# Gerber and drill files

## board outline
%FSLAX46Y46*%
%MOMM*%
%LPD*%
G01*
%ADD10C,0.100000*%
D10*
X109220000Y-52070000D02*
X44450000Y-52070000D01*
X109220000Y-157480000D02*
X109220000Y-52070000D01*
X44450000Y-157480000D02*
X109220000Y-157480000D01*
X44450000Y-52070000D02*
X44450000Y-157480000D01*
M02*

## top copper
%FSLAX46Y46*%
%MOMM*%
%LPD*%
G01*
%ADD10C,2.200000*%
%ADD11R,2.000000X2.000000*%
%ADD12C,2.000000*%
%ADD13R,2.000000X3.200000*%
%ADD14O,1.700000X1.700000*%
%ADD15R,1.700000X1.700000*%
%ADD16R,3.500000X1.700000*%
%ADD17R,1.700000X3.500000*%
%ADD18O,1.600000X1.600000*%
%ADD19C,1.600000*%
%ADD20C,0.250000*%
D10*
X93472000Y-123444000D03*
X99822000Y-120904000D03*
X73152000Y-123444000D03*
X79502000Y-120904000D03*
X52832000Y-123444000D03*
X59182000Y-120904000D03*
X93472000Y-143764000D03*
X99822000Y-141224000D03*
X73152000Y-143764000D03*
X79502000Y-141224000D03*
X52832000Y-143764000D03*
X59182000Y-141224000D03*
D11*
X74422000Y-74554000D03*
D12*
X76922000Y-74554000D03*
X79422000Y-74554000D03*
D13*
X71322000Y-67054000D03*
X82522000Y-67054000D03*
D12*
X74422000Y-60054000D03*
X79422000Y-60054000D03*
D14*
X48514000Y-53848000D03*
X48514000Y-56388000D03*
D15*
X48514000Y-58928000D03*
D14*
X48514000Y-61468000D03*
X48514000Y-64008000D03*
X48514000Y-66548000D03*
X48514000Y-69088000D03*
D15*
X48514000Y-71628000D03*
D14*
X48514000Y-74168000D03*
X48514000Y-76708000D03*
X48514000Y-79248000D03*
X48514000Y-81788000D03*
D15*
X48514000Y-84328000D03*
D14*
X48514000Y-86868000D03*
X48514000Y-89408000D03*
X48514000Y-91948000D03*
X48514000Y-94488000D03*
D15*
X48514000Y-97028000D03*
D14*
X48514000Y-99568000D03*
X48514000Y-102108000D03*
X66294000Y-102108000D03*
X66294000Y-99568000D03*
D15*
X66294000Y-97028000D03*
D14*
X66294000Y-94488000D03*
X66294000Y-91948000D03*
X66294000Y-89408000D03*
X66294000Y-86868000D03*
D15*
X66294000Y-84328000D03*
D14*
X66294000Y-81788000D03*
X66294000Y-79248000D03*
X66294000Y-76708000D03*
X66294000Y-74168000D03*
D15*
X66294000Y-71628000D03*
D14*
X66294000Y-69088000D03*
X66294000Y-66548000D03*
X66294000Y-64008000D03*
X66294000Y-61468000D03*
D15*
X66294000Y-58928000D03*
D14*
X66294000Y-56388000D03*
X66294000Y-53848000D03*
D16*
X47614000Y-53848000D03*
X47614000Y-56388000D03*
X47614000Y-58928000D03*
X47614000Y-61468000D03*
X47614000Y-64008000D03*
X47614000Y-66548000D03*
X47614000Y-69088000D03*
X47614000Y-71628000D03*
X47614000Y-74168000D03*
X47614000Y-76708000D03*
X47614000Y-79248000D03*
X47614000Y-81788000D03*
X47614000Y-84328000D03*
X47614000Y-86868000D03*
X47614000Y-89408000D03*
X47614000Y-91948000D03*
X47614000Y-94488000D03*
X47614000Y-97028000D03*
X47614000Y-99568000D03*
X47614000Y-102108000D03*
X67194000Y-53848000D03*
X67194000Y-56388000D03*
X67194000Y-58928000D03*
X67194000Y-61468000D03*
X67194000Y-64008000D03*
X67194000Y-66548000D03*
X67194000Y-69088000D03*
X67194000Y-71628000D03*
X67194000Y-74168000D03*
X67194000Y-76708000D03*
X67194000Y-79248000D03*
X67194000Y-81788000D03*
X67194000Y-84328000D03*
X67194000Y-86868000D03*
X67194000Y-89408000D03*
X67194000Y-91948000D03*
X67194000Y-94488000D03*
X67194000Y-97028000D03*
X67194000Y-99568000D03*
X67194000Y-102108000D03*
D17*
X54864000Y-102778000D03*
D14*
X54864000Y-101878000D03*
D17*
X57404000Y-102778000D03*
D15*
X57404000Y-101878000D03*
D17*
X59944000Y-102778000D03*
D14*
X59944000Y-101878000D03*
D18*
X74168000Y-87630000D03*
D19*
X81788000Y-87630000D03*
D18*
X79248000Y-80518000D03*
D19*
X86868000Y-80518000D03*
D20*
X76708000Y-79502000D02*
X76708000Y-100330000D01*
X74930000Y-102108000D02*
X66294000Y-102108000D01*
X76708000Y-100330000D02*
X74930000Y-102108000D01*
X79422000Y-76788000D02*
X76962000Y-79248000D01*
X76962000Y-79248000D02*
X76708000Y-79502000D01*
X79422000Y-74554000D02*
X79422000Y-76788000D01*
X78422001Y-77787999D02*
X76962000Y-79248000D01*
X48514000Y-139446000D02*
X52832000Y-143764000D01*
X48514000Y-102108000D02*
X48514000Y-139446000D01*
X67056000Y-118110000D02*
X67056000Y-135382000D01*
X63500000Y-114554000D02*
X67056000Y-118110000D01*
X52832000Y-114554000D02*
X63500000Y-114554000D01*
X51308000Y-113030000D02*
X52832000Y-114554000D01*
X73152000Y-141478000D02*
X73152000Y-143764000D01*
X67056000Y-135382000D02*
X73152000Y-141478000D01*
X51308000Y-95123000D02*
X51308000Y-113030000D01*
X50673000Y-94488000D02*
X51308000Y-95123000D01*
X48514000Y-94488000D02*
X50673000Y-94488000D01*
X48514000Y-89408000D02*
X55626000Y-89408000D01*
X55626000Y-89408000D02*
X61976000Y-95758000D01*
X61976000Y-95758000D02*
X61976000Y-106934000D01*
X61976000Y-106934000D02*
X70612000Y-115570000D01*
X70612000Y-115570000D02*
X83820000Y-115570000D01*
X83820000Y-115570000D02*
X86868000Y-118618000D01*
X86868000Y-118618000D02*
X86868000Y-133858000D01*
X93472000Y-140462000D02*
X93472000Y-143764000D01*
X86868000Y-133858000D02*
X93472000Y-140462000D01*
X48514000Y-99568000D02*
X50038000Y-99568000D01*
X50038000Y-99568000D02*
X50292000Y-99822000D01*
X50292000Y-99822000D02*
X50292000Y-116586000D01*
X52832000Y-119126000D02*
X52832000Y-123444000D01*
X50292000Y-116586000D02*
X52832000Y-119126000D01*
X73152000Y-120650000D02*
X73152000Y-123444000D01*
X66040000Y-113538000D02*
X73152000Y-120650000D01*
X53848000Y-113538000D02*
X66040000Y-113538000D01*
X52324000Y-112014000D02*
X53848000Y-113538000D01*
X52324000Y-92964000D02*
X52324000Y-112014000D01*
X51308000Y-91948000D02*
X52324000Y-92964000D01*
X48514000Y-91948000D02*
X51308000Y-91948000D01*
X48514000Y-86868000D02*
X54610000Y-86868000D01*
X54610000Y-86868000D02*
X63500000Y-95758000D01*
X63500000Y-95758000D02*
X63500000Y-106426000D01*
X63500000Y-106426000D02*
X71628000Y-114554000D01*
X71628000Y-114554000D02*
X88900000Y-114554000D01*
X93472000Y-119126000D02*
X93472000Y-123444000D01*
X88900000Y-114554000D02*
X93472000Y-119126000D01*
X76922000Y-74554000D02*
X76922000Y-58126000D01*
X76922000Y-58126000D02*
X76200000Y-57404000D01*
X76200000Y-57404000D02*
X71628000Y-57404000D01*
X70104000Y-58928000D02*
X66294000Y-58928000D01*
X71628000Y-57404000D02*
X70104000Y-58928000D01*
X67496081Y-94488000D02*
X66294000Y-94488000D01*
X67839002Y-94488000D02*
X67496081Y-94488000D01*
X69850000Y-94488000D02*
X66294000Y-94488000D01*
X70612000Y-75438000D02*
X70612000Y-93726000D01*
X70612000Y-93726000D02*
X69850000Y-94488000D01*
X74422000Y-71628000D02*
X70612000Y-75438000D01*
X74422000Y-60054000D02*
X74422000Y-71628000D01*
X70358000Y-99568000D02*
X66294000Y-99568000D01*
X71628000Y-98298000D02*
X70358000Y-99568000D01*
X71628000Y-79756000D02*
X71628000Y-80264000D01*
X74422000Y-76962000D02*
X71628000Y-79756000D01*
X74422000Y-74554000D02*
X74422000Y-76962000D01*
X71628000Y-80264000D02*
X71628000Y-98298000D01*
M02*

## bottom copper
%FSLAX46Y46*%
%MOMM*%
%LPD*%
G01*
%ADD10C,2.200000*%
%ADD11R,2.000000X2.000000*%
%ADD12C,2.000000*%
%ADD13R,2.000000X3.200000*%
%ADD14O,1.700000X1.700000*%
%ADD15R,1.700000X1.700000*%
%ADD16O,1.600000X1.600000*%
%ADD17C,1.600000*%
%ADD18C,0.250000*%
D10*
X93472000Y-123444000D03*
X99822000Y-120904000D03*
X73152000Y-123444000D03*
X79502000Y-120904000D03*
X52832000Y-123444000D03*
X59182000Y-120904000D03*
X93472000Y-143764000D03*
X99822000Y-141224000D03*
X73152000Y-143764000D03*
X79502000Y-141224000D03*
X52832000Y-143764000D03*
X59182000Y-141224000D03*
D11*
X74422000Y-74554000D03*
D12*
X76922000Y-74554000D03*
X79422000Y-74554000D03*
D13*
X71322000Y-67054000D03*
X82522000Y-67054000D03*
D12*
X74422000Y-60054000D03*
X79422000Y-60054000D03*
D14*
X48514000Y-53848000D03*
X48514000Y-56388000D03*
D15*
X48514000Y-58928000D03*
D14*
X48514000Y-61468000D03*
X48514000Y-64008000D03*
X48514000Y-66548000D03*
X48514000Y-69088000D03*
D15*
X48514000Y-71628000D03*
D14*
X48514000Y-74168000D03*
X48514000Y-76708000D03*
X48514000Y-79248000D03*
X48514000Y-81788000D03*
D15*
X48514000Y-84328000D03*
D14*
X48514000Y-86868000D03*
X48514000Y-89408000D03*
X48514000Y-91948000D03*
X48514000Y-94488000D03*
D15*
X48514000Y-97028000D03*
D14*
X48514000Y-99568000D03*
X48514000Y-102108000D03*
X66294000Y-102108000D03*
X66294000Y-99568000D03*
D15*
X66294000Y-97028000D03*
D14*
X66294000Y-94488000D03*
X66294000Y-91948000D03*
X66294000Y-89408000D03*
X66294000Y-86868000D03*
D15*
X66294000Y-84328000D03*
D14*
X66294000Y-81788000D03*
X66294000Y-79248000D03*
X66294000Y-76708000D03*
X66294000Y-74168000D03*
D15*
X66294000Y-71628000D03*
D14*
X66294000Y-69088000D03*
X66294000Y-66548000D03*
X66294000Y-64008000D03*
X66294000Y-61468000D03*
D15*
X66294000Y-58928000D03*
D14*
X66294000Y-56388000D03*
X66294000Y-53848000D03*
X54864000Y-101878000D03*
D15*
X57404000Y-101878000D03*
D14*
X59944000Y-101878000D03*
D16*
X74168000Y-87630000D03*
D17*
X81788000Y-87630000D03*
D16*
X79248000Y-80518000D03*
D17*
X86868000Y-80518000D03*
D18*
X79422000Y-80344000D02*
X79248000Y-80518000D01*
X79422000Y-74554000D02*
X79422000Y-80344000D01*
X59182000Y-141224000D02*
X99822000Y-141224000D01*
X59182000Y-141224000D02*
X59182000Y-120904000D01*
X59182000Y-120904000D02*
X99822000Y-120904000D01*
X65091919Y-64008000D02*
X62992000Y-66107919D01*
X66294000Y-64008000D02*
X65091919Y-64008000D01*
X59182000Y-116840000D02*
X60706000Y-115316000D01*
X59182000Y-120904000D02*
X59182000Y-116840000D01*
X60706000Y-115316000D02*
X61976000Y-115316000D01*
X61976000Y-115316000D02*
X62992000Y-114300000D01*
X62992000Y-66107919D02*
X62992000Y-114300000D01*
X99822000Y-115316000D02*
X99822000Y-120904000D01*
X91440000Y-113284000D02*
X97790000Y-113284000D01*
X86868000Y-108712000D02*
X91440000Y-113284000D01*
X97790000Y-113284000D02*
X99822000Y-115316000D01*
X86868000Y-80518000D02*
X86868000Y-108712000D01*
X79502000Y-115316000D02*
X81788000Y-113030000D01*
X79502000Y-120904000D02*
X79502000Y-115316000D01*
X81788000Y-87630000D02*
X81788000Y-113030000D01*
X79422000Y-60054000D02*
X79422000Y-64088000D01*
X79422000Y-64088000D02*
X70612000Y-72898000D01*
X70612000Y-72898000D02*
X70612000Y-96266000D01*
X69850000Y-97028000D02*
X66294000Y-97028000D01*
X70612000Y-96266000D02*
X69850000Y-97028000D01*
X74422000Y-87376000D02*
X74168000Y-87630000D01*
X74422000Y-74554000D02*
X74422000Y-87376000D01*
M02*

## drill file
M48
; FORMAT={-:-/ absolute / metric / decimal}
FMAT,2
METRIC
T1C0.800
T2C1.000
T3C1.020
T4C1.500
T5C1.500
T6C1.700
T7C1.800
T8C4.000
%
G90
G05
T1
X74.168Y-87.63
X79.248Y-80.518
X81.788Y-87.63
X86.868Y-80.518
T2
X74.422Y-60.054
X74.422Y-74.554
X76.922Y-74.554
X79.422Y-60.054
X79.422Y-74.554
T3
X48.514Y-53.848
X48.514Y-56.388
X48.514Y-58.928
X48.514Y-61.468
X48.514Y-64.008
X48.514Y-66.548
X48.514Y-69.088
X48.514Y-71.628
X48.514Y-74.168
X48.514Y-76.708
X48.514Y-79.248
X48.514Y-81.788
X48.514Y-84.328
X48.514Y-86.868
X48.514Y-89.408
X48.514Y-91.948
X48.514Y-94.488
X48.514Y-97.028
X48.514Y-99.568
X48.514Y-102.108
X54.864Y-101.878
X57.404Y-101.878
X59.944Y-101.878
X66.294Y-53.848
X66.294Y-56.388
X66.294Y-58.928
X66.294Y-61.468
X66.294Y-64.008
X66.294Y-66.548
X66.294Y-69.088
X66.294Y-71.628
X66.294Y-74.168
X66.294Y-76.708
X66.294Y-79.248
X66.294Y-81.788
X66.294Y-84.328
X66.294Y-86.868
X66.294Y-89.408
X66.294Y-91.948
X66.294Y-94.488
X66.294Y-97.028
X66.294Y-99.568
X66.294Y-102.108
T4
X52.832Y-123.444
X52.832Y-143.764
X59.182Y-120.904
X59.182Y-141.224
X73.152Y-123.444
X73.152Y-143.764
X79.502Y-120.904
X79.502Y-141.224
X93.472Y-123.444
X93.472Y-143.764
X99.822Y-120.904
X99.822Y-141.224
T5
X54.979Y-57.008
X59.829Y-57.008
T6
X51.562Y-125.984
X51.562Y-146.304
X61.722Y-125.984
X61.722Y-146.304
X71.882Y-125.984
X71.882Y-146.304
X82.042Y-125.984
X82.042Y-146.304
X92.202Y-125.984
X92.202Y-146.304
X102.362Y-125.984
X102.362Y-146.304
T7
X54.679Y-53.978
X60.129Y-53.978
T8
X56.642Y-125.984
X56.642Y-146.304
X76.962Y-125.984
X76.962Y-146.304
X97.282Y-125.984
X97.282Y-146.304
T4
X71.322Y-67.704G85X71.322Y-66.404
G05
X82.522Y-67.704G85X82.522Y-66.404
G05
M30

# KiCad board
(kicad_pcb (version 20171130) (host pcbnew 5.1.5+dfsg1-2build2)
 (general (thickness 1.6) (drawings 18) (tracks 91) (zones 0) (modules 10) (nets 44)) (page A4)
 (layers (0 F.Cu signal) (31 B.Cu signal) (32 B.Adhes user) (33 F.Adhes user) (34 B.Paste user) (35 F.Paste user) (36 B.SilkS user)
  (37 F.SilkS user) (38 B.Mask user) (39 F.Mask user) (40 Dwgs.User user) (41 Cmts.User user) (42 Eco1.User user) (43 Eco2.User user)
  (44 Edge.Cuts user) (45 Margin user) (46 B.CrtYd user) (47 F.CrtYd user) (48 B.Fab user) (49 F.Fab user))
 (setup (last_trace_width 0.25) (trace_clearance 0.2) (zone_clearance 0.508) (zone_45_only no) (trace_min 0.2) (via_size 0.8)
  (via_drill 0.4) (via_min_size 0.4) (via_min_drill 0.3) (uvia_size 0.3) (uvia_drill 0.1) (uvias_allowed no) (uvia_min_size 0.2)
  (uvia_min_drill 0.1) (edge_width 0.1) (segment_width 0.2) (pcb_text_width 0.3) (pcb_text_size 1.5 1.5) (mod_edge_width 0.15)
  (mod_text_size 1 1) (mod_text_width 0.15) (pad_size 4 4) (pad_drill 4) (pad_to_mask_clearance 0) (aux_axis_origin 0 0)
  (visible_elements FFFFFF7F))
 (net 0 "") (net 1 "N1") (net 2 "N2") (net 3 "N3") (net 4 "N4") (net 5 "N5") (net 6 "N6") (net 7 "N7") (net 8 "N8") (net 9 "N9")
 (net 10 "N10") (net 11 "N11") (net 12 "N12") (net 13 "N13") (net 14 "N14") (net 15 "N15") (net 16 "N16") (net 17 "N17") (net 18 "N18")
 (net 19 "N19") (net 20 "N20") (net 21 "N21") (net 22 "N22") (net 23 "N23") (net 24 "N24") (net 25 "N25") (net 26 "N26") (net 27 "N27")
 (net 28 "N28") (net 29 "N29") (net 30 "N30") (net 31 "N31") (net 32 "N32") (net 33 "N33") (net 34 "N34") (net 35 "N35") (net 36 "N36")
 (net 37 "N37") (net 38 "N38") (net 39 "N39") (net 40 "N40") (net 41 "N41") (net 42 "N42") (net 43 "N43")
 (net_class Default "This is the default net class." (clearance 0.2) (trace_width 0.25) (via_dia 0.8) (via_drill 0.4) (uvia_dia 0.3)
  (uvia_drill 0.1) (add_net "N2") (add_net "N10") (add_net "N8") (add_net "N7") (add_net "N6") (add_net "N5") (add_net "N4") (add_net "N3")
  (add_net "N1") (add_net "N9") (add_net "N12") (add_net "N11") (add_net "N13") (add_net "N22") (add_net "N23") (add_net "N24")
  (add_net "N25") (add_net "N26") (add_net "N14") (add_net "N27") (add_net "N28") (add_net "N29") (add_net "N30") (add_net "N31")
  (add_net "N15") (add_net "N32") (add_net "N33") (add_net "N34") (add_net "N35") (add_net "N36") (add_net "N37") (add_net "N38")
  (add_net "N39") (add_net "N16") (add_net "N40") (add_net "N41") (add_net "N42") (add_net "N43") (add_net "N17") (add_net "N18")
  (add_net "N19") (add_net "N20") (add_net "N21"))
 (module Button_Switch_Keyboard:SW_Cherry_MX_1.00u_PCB (layer F.Cu) (at 99.822 120.904)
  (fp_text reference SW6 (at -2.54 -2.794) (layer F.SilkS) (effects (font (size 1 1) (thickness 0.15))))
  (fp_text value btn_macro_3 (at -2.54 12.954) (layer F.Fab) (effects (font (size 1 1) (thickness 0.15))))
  (pad "" np_thru_hole circle (at 2.54 5.08) (size 1.7 1.7) (drill 1.7) (layers *.Cu *.Mask))
  (pad "" np_thru_hole circle (at -7.62 5.08) (size 1.7 1.7) (drill 1.7) (layers *.Cu *.Mask))
  (pad "" np_thru_hole circle (at -2.54 5.08) (size 4 4) (drill 4) (layers *.Cu *.Mask))
  (pad 2 thru_hole circle (at -6.35 2.54) (size 2.2 2.2) (drill 1.5) (layers *.Cu *.Mask) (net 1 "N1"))
  (pad 1 thru_hole circle (at 0 0) (size 2.2 2.2) (drill 1.5) (layers *.Cu *.Mask) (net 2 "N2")))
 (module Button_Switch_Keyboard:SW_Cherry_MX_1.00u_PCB (layer F.Cu) (at 79.502 120.904)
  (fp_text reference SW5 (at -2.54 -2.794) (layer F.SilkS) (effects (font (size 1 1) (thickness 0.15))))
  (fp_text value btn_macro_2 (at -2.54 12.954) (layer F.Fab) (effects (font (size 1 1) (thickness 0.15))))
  (pad "" np_thru_hole circle (at 2.54 5.08) (size 1.7 1.7) (drill 1.7) (layers *.Cu *.Mask))
  (pad "" np_thru_hole circle (at -7.62 5.08) (size 1.7 1.7) (drill 1.7) (layers *.Cu *.Mask))
  (pad "" np_thru_hole circle (at -2.54 5.08) (size 4 4) (drill 4) (layers *.Cu *.Mask))
  (pad 2 thru_hole circle (at -6.35 2.54) (size 2.2 2.2) (drill 1.5) (layers *.Cu *.Mask) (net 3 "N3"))
  (pad 1 thru_hole circle (at 0 0) (size 2.2 2.2) (drill 1.5) (layers *.Cu *.Mask) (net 2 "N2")))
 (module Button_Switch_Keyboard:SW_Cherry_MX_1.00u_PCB (layer F.Cu) (at 59.182 120.904)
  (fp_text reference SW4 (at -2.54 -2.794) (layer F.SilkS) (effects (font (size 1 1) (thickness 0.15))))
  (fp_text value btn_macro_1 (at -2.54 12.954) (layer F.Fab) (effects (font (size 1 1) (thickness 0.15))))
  (pad "" np_thru_hole circle (at 2.54 5.08) (size 1.7 1.7) (drill 1.7) (layers *.Cu *.Mask))
  (pad "" np_thru_hole circle (at -7.62 5.08) (size 1.7 1.7) (drill 1.7) (layers *.Cu *.Mask))
  (pad "" np_thru_hole circle (at -2.54 5.08) (size 4 4) (drill 4) (layers *.Cu *.Mask))
  (pad 2 thru_hole circle (at -6.35 2.54) (size 2.2 2.2) (drill 1.5) (layers *.Cu *.Mask) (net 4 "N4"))
  (pad 1 thru_hole circle (at 0 0) (size 2.2 2.2) (drill 1.5) (layers *.Cu *.Mask) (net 2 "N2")))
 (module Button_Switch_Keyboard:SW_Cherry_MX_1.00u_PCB (layer F.Cu) (at 99.822 141.224)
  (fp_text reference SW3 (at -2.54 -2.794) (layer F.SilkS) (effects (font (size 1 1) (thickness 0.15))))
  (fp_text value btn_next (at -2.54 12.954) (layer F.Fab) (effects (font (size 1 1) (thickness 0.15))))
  (pad "" np_thru_hole circle (at 2.54 5.08) (size 1.7 1.7) (drill 1.7) (layers *.Cu *.Mask))
  (pad "" np_thru_hole circle (at -7.62 5.08) (size 1.7 1.7) (drill 1.7) (layers *.Cu *.Mask))
  (pad "" np_thru_hole circle (at -2.54 5.08) (size 4 4) (drill 4) (layers *.Cu *.Mask))
  (pad 2 thru_hole circle (at -6.35 2.54) (size 2.2 2.2) (drill 1.5) (layers *.Cu *.Mask) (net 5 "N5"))
  (pad 1 thru_hole circle (at 0 0) (size 2.2 2.2) (drill 1.5) (layers *.Cu *.Mask) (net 2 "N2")))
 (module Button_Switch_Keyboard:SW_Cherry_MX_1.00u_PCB (layer F.Cu) (at 79.502 141.224)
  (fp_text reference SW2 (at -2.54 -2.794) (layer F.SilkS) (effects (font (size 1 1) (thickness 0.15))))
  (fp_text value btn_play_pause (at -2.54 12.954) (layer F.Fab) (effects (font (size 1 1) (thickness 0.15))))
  (pad "" np_thru_hole circle (at 2.54 5.08) (size 1.7 1.7) (drill 1.7) (layers *.Cu *.Mask))
  (pad "" np_thru_hole circle (at -7.62 5.08) (size 1.7 1.7) (drill 1.7) (layers *.Cu *.Mask))
  (pad "" np_thru_hole circle (at -2.54 5.08) (size 4 4) (drill 4) (layers *.Cu *.Mask))
  (pad 2 thru_hole circle (at -6.35 2.54) (size 2.2 2.2) (drill 1.5) (layers *.Cu *.Mask) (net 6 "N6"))
  (pad 1 thru_hole circle (at 0 0) (size 2.2 2.2) (drill 1.5) (layers *.Cu *.Mask) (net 2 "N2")))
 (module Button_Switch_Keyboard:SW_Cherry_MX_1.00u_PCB (layer F.Cu) (at 59.182 141.224)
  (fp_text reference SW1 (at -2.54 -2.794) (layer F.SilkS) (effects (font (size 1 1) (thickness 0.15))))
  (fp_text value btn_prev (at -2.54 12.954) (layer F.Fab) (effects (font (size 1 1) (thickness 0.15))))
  (pad "" np_thru_hole circle (at 2.54 5.08) (size 1.7 1.7) (drill 1.7) (layers *.Cu *.Mask))
  (pad "" np_thru_hole circle (at -7.62 5.08) (size 1.7 1.7) (drill 1.7) (layers *.Cu *.Mask))
  (pad "" np_thru_hole circle (at -2.54 5.08) (size 4 4) (drill 4) (layers *.Cu *.Mask))
  (pad 2 thru_hole circle (at -6.35 2.54) (size 2.2 2.2) (drill 1.5) (layers *.Cu *.Mask) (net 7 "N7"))
  (pad 1 thru_hole circle (at 0 0) (size 2.2 2.2) (drill 1.5) (layers *.Cu *.Mask) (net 2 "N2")))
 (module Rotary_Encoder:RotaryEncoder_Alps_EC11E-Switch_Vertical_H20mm (layer F.Cu) (at 74.422 74.554 90)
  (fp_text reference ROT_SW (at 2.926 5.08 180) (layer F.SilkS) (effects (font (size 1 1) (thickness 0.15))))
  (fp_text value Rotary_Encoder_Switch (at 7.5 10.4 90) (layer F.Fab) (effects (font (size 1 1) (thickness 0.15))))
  (pad A thru_hole rect (at 0 0 90) (size 2 2) (drill 1) (layers *.Cu *.Mask) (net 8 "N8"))
  (pad C thru_hole circle (at 0 2.5 90) (size 2 2) (drill 1) (layers *.Cu *.Mask) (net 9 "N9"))
  (pad B thru_hole circle (at 0 5 90) (size 2 2) (drill 1) (layers *.Cu *.Mask) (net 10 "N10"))
  (pad MP thru_hole rect (at 7.5 -3.1 90) (size 3.2 2) (drill oval 2.8 1.5) (layers *.Cu *.Mask))
  (pad MP thru_hole rect (at 7.5 8.1 90) (size 3.2 2) (drill oval 2.8 1.5) (layers *.Cu *.Mask))
  (pad S2 thru_hole circle (at 14.5 0 90) (size 2 2) (drill 1) (layers *.Cu *.Mask) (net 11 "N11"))
  (pad S1 thru_hole circle (at 14.5 5 90) (size 2 2) (drill 1) (layers *.Cu *.Mask) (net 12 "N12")))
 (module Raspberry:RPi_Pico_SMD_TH (layer F.Cu) (at 57.404 77.978)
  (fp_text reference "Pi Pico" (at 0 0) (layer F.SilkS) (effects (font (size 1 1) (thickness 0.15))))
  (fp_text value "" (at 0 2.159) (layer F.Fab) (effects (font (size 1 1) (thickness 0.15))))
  (pad 1 thru_hole oval (at -8.89 -24.13) (size 1.7 1.7) (drill 1.02) (layers *.Cu *.Mask) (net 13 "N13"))
  (pad 2 thru_hole oval (at -8.89 -21.59) (size 1.7 1.7) (drill 1.02) (layers *.Cu *.Mask) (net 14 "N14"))
  (pad 3 thru_hole rect (at -8.89 -19.05) (size 1.7 1.7) (drill 1.02) (layers *.Cu *.Mask) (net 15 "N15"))
  (pad 4 thru_hole oval (at -8.89 -16.51) (size 1.7 1.7) (drill 1.02) (layers *.Cu *.Mask) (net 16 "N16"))
  (pad 5 thru_hole oval (at -8.89 -13.97) (size 1.7 1.7) (drill 1.02) (layers *.Cu *.Mask) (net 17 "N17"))
  (pad 6 thru_hole oval (at -8.89 -11.43) (size 1.7 1.7) (drill 1.02) (layers *.Cu *.Mask) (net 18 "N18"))
  (pad 7 thru_hole oval (at -8.89 -8.89) (size 1.7 1.7) (drill 1.02) (layers *.Cu *.Mask) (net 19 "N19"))
  (pad 8 thru_hole rect (at -8.89 -6.35) (size 1.7 1.7) (drill 1.02) (layers *.Cu *.Mask) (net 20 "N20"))
  (pad 9 thru_hole oval (at -8.89 -3.81) (size 1.7 1.7) (drill 1.02) (layers *.Cu *.Mask) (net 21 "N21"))
  (pad 10 thru_hole oval (at -8.89 -1.27) (size 1.7 1.7) (drill 1.02) (layers *.Cu *.Mask) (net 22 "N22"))
  (pad 11 thru_hole oval (at -8.89 1.27) (size 1.7 1.7) (drill 1.02) (layers *.Cu *.Mask) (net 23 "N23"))
  (pad 12 thru_hole oval (at -8.89 3.81) (size 1.7 1.7) (drill 1.02) (layers *.Cu *.Mask) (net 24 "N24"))
  (pad 13 thru_hole rect (at -8.89 6.35) (size 1.7 1.7) (drill 1.02) (layers *.Cu *.Mask) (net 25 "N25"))
  (pad 14 thru_hole oval (at -8.89 8.89) (size 1.7 1.7) (drill 1.02) (layers *.Cu *.Mask) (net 1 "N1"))
  (pad 15 thru_hole oval (at -8.89 11.43) (size 1.7 1.7) (drill 1.02) (layers *.Cu *.Mask) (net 5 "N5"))
  (pad 16 thru_hole oval (at -8.89 13.97) (size 1.7 1.7) (drill 1.02) (layers *.Cu *.Mask) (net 3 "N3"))
  (pad 17 thru_hole oval (at -8.89 16.51) (size 1.7 1.7) (drill 1.02) (layers *.Cu *.Mask) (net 6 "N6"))
  (pad 18 thru_hole rect (at -8.89 19.05) (size 1.7 1.7) (drill 1.02) (layers *.Cu *.Mask) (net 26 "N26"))
  (pad 19 thru_hole oval (at -8.89 21.59) (size 1.7 1.7) (drill 1.02) (layers *.Cu *.Mask) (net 4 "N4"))
  (pad 20 thru_hole oval (at -8.89 24.13) (size 1.7 1.7) (drill 1.02) (layers *.Cu *.Mask) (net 7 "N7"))
  (pad 21 thru_hole oval (at 8.89 24.13) (size 1.7 1.7) (drill 1.02) (layers *.Cu *.Mask) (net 10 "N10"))
  (pad 22 thru_hole oval (at 8.89 21.59) (size 1.7 1.7) (drill 1.02) (layers *.Cu *.Mask) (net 8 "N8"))
  (pad 23 thru_hole rect (at 8.89 19.05) (size 1.7 1.7) (drill 1.02) (layers *.Cu *.Mask) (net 12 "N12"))
  (pad 24 thru_hole oval (at 8.89 16.51) (size 1.7 1.7) (drill 1.02) (layers *.Cu *.Mask) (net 11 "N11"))
  (pad 25 thru_hole oval (at 8.89 13.97) (size 1.7 1.7) (drill 1.02) (layers *.Cu *.Mask) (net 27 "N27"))
  (pad 26 thru_hole oval (at 8.89 11.43) (size 1.7 1.7) (drill 1.02) (layers *.Cu *.Mask) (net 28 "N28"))
  (pad 27 thru_hole oval (at 8.89 8.89) (size 1.7 1.7) (drill 1.02) (layers *.Cu *.Mask) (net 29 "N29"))
  (pad 28 thru_hole rect (at 8.89 6.35) (size 1.7 1.7) (drill 1.02) (layers *.Cu *.Mask) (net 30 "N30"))
  (pad 29 thru_hole oval (at 8.89 3.81) (size 1.7 1.7) (drill 1.02) (layers *.Cu *.Mask) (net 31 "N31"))
  (pad 30 thru_hole oval (at 8.89 1.27) (size 1.7 1.7) (drill 1.02) (layers *.Cu *.Mask) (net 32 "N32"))
  (pad 31 thru_hole oval (at 8.89 -1.27) (size 1.7 1.7) (drill 1.02) (layers *.Cu *.Mask) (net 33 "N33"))
  (pad 32 thru_hole oval (at 8.89 -3.81) (size 1.7 1.7) (drill 1.02) (layers *.Cu *.Mask) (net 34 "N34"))
  (pad 33 thru_hole rect (at 8.89 -6.35) (size 1.7 1.7) (drill 1.02) (layers *.Cu *.Mask) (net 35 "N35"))
  (pad 34 thru_hole oval (at 8.89 -8.89) (size 1.7 1.7) (drill 1.02) (layers *.Cu *.Mask) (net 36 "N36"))
  (pad 35 thru_hole oval (at 8.89 -11.43) (size 1.7 1.7) (drill 1.02) (layers *.Cu *.Mask) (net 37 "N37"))
  (pad 36 thru_hole oval (at 8.89 -13.97) (size 1.7 1.7) (drill 1.02) (layers *.Cu *.Mask) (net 2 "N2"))
  (pad 37 thru_hole oval (at 8.89 -16.51) (size 1.7 1.7) (drill 1.02) (layers *.Cu *.Mask) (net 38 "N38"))
  (pad 38 thru_hole rect (at 8.89 -19.05) (size 1.7 1.7) (drill 1.02) (layers *.Cu *.Mask) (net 9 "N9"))
  (pad 39 thru_hole oval (at 8.89 -21.59) (size 1.7 1.7) (drill 1.02) (layers *.Cu *.Mask) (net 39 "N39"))
  (pad 40 thru_hole oval (at 8.89 -24.13) (size 1.7 1.7) (drill 1.02) (layers *.Cu *.Mask) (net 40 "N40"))
  (pad 1 smd rect (at -8.89 -24.13) (size 3.5 1.7) (drill (offset -0.9 0)) (layers F.Cu F.Mask) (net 13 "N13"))
  (pad 2 smd rect (at -8.89 -21.59) (size 3.5 1.7) (drill (offset -0.9 0)) (layers F.Cu F.Mask) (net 14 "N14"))
  (pad 3 smd rect (at -8.89 -19.05) (size 3.5 1.7) (drill (offset -0.9 0)) (layers F.Cu F.Mask) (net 15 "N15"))
  (pad 4 smd rect (at -8.89 -16.51) (size 3.5 1.7) (drill (offset -0.9 0)) (layers F.Cu F.Mask) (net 16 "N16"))
  (pad 5 smd rect (at -8.89 -13.97) (size 3.5 1.7) (drill (offset -0.9 0)) (layers F.Cu F.Mask) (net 17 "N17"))
  (pad 6 smd rect (at -8.89 -11.43) (size 3.5 1.7) (drill (offset -0.9 0)) (layers F.Cu F.Mask) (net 18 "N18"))
  (pad 7 smd rect (at -8.89 -8.89) (size 3.5 1.7) (drill (offset -0.9 0)) (layers F.Cu F.Mask) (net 19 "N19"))
  (pad 8 smd rect (at -8.89 -6.35) (size 3.5 1.7) (drill (offset -0.9 0)) (layers F.Cu F.Mask) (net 20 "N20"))
  (pad 9 smd rect (at -8.89 -3.81) (size 3.5 1.7) (drill (offset -0.9 0)) (layers F.Cu F.Mask) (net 21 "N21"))
  (pad 10 smd rect (at -8.89 -1.27) (size 3.5 1.7) (drill (offset -0.9 0)) (layers F.Cu F.Mask) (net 22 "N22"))
  (pad 11 smd rect (at -8.89 1.27) (size 3.5 1.7) (drill (offset -0.9 0)) (layers F.Cu F.Mask) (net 23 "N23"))
  (pad 12 smd rect (at -8.89 3.81) (size 3.5 1.7) (drill (offset -0.9 0)) (layers F.Cu F.Mask) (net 24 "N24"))
  (pad 13 smd rect (at -8.89 6.35) (size 3.5 1.7) (drill (offset -0.9 0)) (layers F.Cu F.Mask) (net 25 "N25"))
  (pad 14 smd rect (at -8.89 8.89) (size 3.5 1.7) (drill (offset -0.9 0)) (layers F.Cu F.Mask) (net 1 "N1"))
  (pad 15 smd rect (at -8.89 11.43) (size 3.5 1.7) (drill (offset -0.9 0)) (layers F.Cu F.Mask) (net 5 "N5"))
  (pad 16 smd rect (at -8.89 13.97) (size 3.5 1.7) (drill (offset -0.9 0)) (layers F.Cu F.Mask) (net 3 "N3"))
  (pad 17 smd rect (at -8.89 16.51) (size 3.5 1.7) (drill (offset -0.9 0)) (layers F.Cu F.Mask) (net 6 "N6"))
  (pad 18 smd rect (at -8.89 19.05) (size 3.5 1.7) (drill (offset -0.9 0)) (layers F.Cu F.Mask) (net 26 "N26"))
  (pad 19 smd rect (at -8.89 21.59) (size 3.5 1.7) (drill (offset -0.9 0)) (layers F.Cu F.Mask) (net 4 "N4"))
  (pad 20 smd rect (at -8.89 24.13) (size 3.5 1.7) (drill (offset -0.9 0)) (layers F.Cu F.Mask) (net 7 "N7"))
  (pad 40 smd rect (at 8.89 -24.13) (size 3.5 1.7) (drill (offset 0.9 0)) (layers F.Cu F.Mask) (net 40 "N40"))
  (pad 39 smd rect (at 8.89 -21.59) (size 3.5 1.7) (drill (offset 0.9 0)) (layers F.Cu F.Mask) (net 39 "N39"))
  (pad 38 smd rect (at 8.89 -19.05) (size 3.5 1.7) (drill (offset 0.9 0)) (layers F.Cu F.Mask) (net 9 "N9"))
  (pad 37 smd rect (at 8.89 -16.51) (size 3.5 1.7) (drill (offset 0.9 0)) (layers F.Cu F.Mask) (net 38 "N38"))
  (pad 36 smd rect (at 8.89 -13.97) (size 3.5 1.7) (drill (offset 0.9 0)) (layers F.Cu F.Mask) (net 2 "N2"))
  (pad 35 smd rect (at 8.89 -11.43) (size 3.5 1.7) (drill (offset 0.9 0)) (layers F.Cu F.Mask) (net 37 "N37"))
  (pad 34 smd rect (at 8.89 -8.89) (size 3.5 1.7) (drill (offset 0.9 0)) (layers F.Cu F.Mask) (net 36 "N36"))
  (pad 33 smd rect (at 8.89 -6.35) (size 3.5 1.7) (drill (offset 0.9 0)) (layers F.Cu F.Mask) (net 35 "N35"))
  (pad 32 smd rect (at 8.89 -3.81) (size 3.5 1.7) (drill (offset 0.9 0)) (layers F.Cu F.Mask) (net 34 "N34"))
  (pad 31 smd rect (at 8.89 -1.27) (size 3.5 1.7) (drill (offset 0.9 0)) (layers F.Cu F.Mask) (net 33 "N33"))
  (pad 30 smd rect (at 8.89 1.27) (size 3.5 1.7) (drill (offset 0.9 0)) (layers F.Cu F.Mask) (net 32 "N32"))
  (pad 29 smd rect (at 8.89 3.81) (size 3.5 1.7) (drill (offset 0.9 0)) (layers F.Cu F.Mask) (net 31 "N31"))
  (pad 28 smd rect (at 8.89 6.35) (size 3.5 1.7) (drill (offset 0.9 0)) (layers F.Cu F.Mask) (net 30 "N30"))
  (pad 27 smd rect (at 8.89 8.89) (size 3.5 1.7) (drill (offset 0.9 0)) (layers F.Cu F.Mask) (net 29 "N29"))
  (pad 26 smd rect (at 8.89 11.43) (size 3.5 1.7) (drill (offset 0.9 0)) (layers F.Cu F.Mask) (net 28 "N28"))
  (pad 25 smd rect (at 8.89 13.97) (size 3.5 1.7) (drill (offset 0.9 0)) (layers F.Cu F.Mask) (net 27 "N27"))
  (pad 24 smd rect (at 8.89 16.51) (size 3.5 1.7) (drill (offset 0.9 0)) (layers F.Cu F.Mask) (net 11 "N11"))
  (pad 23 smd rect (at 8.89 19.05) (size 3.5 1.7) (drill (offset 0.9 0)) (layers F.Cu F.Mask) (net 12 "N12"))
  (pad 22 smd rect (at 8.89 21.59) (size 3.5 1.7) (drill (offset 0.9 0)) (layers F.Cu F.Mask) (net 8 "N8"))
  (pad 21 smd rect (at 8.89 24.13) (size 3.5 1.7) (drill (offset 0.9 0)) (layers F.Cu F.Mask) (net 10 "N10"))
  (pad "" np_thru_hole oval (at -2.725 -24) (size 1.8 1.8) (drill 1.8) (layers *.Cu *.Mask))
  (pad "" np_thru_hole oval (at 2.725 -24) (size 1.8 1.8) (drill 1.8) (layers *.Cu *.Mask))
  (pad "" np_thru_hole oval (at -2.425 -20.97) (size 1.5 1.5) (drill 1.5) (layers *.Cu *.Mask))
  (pad "" np_thru_hole oval (at 2.425 -20.97) (size 1.5 1.5) (drill 1.5) (layers *.Cu *.Mask))
  (pad 41 smd rect (at -2.54 23.9 90) (size 3.5 1.7) (drill (offset -0.9 0)) (layers F.Cu F.Mask) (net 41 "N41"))
  (pad 41 thru_hole oval (at -2.54 23.9) (size 1.7 1.7) (drill 1.02) (layers *.Cu *.Mask) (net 41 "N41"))
  (pad 42 smd rect (at 0 23.9 90) (size 3.5 1.7) (drill (offset -0.9 0)) (layers F.Cu F.Mask) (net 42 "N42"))
  (pad 42 thru_hole rect (at 0 23.9) (size 1.7 1.7) (drill 1.02) (layers *.Cu *.Mask) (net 42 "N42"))
  (pad 43 smd rect (at 2.54 23.9 90) (size 3.5 1.7) (drill (offset -0.9 0)) (layers F.Cu F.Mask) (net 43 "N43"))
  (pad 43 thru_hole oval (at 2.54 23.9) (size 1.7 1.7) (drill 1.02) (layers *.Cu *.Mask) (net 43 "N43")))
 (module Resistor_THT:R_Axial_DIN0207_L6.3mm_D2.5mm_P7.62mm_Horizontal (layer F.Cu) (at 81.788 87.63 180)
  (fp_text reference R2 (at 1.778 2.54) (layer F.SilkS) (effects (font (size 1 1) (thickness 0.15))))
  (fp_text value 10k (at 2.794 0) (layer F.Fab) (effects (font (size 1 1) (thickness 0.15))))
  (pad 2 thru_hole oval (at 7.62 0 180) (size 1.6 1.6) (drill 0.8) (layers *.Cu *.Mask) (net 8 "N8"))
  (pad 1 thru_hole circle (at 0 0 180) (size 1.6 1.6) (drill 0.8) (layers *.Cu *.Mask) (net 2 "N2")))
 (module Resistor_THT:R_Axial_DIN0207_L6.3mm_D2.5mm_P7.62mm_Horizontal (layer F.Cu) (at 86.868 80.518 180)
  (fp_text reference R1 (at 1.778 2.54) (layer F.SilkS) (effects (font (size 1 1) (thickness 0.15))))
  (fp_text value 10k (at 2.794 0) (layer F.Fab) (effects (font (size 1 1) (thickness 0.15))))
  (pad 2 thru_hole oval (at 7.62 0 180) (size 1.6 1.6) (drill 0.8) (layers *.Cu *.Mask) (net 10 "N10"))
  (pad 1 thru_hole circle (at 0 0 180) (size 1.6 1.6) (drill 0.8) (layers *.Cu *.Mask) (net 2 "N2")))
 (gr_line (start 109.22 52.07) (end 44.45 52.07) (layer Edge.Cuts) (width 0.1))
 (gr_line (start 109.22 157.48) (end 109.22 52.07) (layer Edge.Cuts) (width 0.1))
 (gr_line (start 44.45 157.48) (end 109.22 157.48) (layer Edge.Cuts) (width 0.1))
 (gr_line (start 44.45 52.07) (end 44.45 157.48) (layer Edge.Cuts) (width 0.1))
 (segment (start 79.422 80.344) (end 79.248 80.518) (width 0.25) (layer B.Cu) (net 10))
 (segment (start 79.422 74.554) (end 79.422 80.344) (width 0.25) (layer B.Cu) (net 10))
 (segment (start 76.708 79.502) (end 76.708 100.33) (width 0.25) (layer F.Cu) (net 10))
 (segment (start 74.93 102.108) (end 66.294 102.108) (width 0.25) (layer F.Cu) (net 10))
 (segment (start 76.708 100.33) (end 74.93 102.108) (width 0.25) (layer F.Cu) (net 10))
 (segment (start 79.422 76.788) (end 76.962 79.248) (width 0.25) (layer F.Cu) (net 10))
 (segment (start 76.962 79.248) (end 76.708 79.502) (width 0.25) (layer F.Cu) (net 10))
 (segment (start 79.422 74.554) (end 79.422 76.788) (width 0.25) (layer F.Cu) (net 10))
 (segment (start 78.422001 77.787999) (end 76.962 79.248) (width 0.25) (layer F.Cu) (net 10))
 (segment (start 59.182 141.224) (end 99.822 141.224) (width 0.25) (layer B.Cu) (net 2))
 (segment (start 59.182 141.224) (end 59.182 120.904) (width 0.25) (layer B.Cu) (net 2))
 (segment (start 59.182 120.904) (end 99.822 120.904) (width 0.25) (layer B.Cu) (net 2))
 (segment (start 65.091919 64.008) (end 62.992 66.107919) (width 0.25) (layer B.Cu) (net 2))
 (segment (start 66.294 64.008) (end 65.091919 64.008) (width 0.25) (layer B.Cu) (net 2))
 (segment (start 59.182 116.84) (end 60.706 115.316) (width 0.25) (layer B.Cu) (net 2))
 (segment (start 59.182 120.904) (end 59.182 116.84) (width 0.25) (layer B.Cu) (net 2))
 (segment (start 60.706 115.316) (end 61.976 115.316) (width 0.25) (layer B.Cu) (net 2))
 (segment (start 61.976 115.316) (end 62.992 114.3) (width 0.25) (layer B.Cu) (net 2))
 (segment (start 62.992 66.107919) (end 62.992 114.3) (width 0.25) (layer B.Cu) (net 2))
 (segment (start 99.822 115.316) (end 99.822 120.904) (width 0.25) (layer B.Cu) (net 2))
 (segment (start 91.44 113.284) (end 97.79 113.284) (width 0.25) (layer B.Cu) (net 2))
 (segment (start 86.868 108.712) (end 91.44 113.284) (width 0.25) (layer B.Cu) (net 2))
 (segment (start 97.79 113.284) (end 99.822 115.316) (width 0.25) (layer B.Cu) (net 2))
 (segment (start 86.868 80.518) (end 86.868 108.712) (width 0.25) (layer B.Cu) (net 2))
 (segment (start 79.502 115.316) (end 81.788 113.03) (width 0.25) (layer B.Cu) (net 2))
 (segment (start 79.502 120.904) (end 79.502 115.316) (width 0.25) (layer B.Cu) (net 2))
 (segment (start 81.788 87.63) (end 81.788 113.03) (width 0.25) (layer B.Cu) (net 2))
 (segment (start 48.514 139.446) (end 52.832 143.764) (width 0.25) (layer F.Cu) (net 7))
 (segment (start 48.514 102.108) (end 48.514 139.446) (width 0.25) (layer F.Cu) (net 7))
 (segment (start 67.056 118.11) (end 67.056 135.382) (width 0.25) (layer F.Cu) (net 6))
 (segment (start 63.5 114.554) (end 67.056 118.11) (width 0.25) (layer F.Cu) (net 6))
 (segment (start 52.832 114.554) (end 63.5 114.554) (width 0.25) (layer F.Cu) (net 6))
 (segment (start 51.308 113.03) (end 52.832 114.554) (width 0.25) (layer F.Cu) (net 6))
 (segment (start 73.152 141.478) (end 73.152 143.764) (width 0.25) (layer F.Cu) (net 6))
 (segment (start 67.056 135.382) (end 73.152 141.478) (width 0.25) (layer F.Cu) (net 6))
 (segment (start 51.308 95.123) (end 51.308 113.03) (width 0.25) (layer F.Cu) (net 6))
 (segment (start 50.673 94.488) (end 51.308 95.123) (width 0.25) (layer F.Cu) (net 6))
 (segment (start 48.514 94.488) (end 50.673 94.488) (width 0.25) (layer F.Cu) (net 6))
 (segment (start 48.514 89.408) (end 55.626 89.408) (width 0.25) (layer F.Cu) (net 5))
 (segment (start 55.626 89.408) (end 61.976 95.758) (width 0.25) (layer F.Cu) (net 5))
 (segment (start 61.976 95.758) (end 61.976 106.934) (width 0.25) (layer F.Cu) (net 5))
 (segment (start 61.976 106.934) (end 70.612 115.57) (width 0.25) (layer F.Cu) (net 5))
 (segment (start 70.612 115.57) (end 83.82 115.57) (width 0.25) (layer F.Cu) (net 5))
 (segment (start 83.82 115.57) (end 86.868 118.618) (width 0.25) (layer F.Cu) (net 5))
 (segment (start 86.868 118.618) (end 86.868 133.858) (width 0.25) (layer F.Cu) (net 5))
 (segment (start 93.472 140.462) (end 93.472 143.764) (width 0.25) (layer F.Cu) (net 5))
 (segment (start 86.868 133.858) (end 93.472 140.462) (width 0.25) (layer F.Cu) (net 5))
 (segment (start 48.514 99.568) (end 50.038 99.568) (width 0.25) (layer F.Cu) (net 4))
 (segment (start 50.038 99.568) (end 50.292 99.822) (width 0.25) (layer F.Cu) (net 4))
 (segment (start 50.292 99.822) (end 50.292 116.586) (width 0.25) (layer F.Cu) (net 4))
 (segment (start 52.832 119.126) (end 52.832 123.444) (width 0.25) (layer F.Cu) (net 4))
 (segment (start 50.292 116.586) (end 52.832 119.126) (width 0.25) (layer F.Cu) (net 4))
 (segment (start 73.152 120.65) (end 73.152 123.444) (width 0.25) (layer F.Cu) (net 3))
 (segment (start 66.04 113.538) (end 73.152 120.65) (width 0.25) (layer F.Cu) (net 3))
 (segment (start 53.848 113.538) (end 66.04 113.538) (width 0.25) (layer F.Cu) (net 3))
 (segment (start 52.324 112.014) (end 53.848 113.538) (width 0.25) (layer F.Cu) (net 3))
 (segment (start 52.324 92.964) (end 52.324 112.014) (width 0.25) (layer F.Cu) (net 3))
 (segment (start 51.308 91.948) (end 52.324 92.964) (width 0.25) (layer F.Cu) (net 3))
 (segment (start 48.514 91.948) (end 51.308 91.948) (width 0.25) (layer F.Cu) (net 3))
 (segment (start 48.514 86.868) (end 54.61 86.868) (width 0.25) (layer F.Cu) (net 1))
 (segment (start 54.61 86.868) (end 63.5 95.758) (width 0.25) (layer F.Cu) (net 1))
 (segment (start 63.5 95.758) (end 63.5 106.426) (width 0.25) (layer F.Cu) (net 1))
 (segment (start 63.5 106.426) (end 71.628 114.554) (width 0.25) (layer F.Cu) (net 1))
 (segment (start 71.628 114.554) (end 88.9 114.554) (width 0.25) (layer F.Cu) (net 1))
 (segment (start 93.472 119.126) (end 93.472 123.444) (width 0.25) (layer F.Cu) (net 1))
 (segment (start 88.9 114.554) (end 93.472 119.126) (width 0.25) (layer F.Cu) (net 1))
 (segment (start 76.922 74.554) (end 76.922 58.126) (width 0.25) (layer F.Cu) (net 9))
 (segment (start 76.922 58.126) (end 76.2 57.404) (width 0.25) (layer F.Cu) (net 9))
 (segment (start 76.2 57.404) (end 71.628 57.404) (width 0.25) (layer F.Cu) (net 9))
 (segment (start 70.104 58.928) (end 66.294 58.928) (width 0.25) (layer F.Cu) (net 9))
 (segment (start 71.628 57.404) (end 70.104 58.928) (width 0.25) (layer F.Cu) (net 9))
 (segment (start 67.496081 94.488) (end 66.294 94.488) (width 0.25) (layer F.Cu) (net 11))
 (segment (start 67.839002 94.488) (end 67.496081 94.488) (width 0.25) (layer F.Cu) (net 11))
 (segment (start 69.85 94.488) (end 66.294 94.488) (width 0.25) (layer F.Cu) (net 11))
 (segment (start 70.612 75.438) (end 70.612 93.726) (width 0.25) (layer F.Cu) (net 11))
 (segment (start 70.612 93.726) (end 69.85 94.488) (width 0.25) (layer F.Cu) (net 11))
 (segment (start 74.422 71.628) (end 70.612 75.438) (width 0.25) (layer F.Cu) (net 11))
 (segment (start 74.422 60.054) (end 74.422 71.628) (width 0.25) (layer F.Cu) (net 11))
 (segment (start 79.422 60.054) (end 79.422 64.088) (width 0.25) (layer B.Cu) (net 12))
 (segment (start 79.422 64.088) (end 70.612 72.898) (width 0.25) (layer B.Cu) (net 12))
 (segment (start 70.612 72.898) (end 70.612 96.266) (width 0.25) (layer B.Cu) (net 12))
 (segment (start 69.85 97.028) (end 66.294 97.028) (width 0.25) (layer B.Cu) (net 12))
 (segment (start 70.612 96.266) (end 69.85 97.028) (width 0.25) (layer B.Cu) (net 12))
 (segment (start 74.422 87.376) (end 74.168 87.63) (width 0.25) (layer B.Cu) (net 8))
 (segment (start 74.422 74.554) (end 74.422 87.376) (width 0.25) (layer B.Cu) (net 8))
 (segment (start 70.358 99.568) (end 66.294 99.568) (width 0.25) (layer F.Cu) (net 8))
 (segment (start 71.628 98.298) (end 70.358 99.568) (width 0.25) (layer F.Cu) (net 8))
 (segment (start 71.628 79.756) (end 71.628 80.264) (width 0.25) (layer F.Cu) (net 8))
 (segment (start 74.422 76.962) (end 71.628 79.756) (width 0.25) (layer F.Cu) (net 8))
 (segment (start 74.422 74.554) (end 74.422 76.962) (width 0.25) (layer F.Cu) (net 8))
 (segment (start 71.628 80.264) (end 71.628 98.298) (width 0.25) (layer F.Cu) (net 8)))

